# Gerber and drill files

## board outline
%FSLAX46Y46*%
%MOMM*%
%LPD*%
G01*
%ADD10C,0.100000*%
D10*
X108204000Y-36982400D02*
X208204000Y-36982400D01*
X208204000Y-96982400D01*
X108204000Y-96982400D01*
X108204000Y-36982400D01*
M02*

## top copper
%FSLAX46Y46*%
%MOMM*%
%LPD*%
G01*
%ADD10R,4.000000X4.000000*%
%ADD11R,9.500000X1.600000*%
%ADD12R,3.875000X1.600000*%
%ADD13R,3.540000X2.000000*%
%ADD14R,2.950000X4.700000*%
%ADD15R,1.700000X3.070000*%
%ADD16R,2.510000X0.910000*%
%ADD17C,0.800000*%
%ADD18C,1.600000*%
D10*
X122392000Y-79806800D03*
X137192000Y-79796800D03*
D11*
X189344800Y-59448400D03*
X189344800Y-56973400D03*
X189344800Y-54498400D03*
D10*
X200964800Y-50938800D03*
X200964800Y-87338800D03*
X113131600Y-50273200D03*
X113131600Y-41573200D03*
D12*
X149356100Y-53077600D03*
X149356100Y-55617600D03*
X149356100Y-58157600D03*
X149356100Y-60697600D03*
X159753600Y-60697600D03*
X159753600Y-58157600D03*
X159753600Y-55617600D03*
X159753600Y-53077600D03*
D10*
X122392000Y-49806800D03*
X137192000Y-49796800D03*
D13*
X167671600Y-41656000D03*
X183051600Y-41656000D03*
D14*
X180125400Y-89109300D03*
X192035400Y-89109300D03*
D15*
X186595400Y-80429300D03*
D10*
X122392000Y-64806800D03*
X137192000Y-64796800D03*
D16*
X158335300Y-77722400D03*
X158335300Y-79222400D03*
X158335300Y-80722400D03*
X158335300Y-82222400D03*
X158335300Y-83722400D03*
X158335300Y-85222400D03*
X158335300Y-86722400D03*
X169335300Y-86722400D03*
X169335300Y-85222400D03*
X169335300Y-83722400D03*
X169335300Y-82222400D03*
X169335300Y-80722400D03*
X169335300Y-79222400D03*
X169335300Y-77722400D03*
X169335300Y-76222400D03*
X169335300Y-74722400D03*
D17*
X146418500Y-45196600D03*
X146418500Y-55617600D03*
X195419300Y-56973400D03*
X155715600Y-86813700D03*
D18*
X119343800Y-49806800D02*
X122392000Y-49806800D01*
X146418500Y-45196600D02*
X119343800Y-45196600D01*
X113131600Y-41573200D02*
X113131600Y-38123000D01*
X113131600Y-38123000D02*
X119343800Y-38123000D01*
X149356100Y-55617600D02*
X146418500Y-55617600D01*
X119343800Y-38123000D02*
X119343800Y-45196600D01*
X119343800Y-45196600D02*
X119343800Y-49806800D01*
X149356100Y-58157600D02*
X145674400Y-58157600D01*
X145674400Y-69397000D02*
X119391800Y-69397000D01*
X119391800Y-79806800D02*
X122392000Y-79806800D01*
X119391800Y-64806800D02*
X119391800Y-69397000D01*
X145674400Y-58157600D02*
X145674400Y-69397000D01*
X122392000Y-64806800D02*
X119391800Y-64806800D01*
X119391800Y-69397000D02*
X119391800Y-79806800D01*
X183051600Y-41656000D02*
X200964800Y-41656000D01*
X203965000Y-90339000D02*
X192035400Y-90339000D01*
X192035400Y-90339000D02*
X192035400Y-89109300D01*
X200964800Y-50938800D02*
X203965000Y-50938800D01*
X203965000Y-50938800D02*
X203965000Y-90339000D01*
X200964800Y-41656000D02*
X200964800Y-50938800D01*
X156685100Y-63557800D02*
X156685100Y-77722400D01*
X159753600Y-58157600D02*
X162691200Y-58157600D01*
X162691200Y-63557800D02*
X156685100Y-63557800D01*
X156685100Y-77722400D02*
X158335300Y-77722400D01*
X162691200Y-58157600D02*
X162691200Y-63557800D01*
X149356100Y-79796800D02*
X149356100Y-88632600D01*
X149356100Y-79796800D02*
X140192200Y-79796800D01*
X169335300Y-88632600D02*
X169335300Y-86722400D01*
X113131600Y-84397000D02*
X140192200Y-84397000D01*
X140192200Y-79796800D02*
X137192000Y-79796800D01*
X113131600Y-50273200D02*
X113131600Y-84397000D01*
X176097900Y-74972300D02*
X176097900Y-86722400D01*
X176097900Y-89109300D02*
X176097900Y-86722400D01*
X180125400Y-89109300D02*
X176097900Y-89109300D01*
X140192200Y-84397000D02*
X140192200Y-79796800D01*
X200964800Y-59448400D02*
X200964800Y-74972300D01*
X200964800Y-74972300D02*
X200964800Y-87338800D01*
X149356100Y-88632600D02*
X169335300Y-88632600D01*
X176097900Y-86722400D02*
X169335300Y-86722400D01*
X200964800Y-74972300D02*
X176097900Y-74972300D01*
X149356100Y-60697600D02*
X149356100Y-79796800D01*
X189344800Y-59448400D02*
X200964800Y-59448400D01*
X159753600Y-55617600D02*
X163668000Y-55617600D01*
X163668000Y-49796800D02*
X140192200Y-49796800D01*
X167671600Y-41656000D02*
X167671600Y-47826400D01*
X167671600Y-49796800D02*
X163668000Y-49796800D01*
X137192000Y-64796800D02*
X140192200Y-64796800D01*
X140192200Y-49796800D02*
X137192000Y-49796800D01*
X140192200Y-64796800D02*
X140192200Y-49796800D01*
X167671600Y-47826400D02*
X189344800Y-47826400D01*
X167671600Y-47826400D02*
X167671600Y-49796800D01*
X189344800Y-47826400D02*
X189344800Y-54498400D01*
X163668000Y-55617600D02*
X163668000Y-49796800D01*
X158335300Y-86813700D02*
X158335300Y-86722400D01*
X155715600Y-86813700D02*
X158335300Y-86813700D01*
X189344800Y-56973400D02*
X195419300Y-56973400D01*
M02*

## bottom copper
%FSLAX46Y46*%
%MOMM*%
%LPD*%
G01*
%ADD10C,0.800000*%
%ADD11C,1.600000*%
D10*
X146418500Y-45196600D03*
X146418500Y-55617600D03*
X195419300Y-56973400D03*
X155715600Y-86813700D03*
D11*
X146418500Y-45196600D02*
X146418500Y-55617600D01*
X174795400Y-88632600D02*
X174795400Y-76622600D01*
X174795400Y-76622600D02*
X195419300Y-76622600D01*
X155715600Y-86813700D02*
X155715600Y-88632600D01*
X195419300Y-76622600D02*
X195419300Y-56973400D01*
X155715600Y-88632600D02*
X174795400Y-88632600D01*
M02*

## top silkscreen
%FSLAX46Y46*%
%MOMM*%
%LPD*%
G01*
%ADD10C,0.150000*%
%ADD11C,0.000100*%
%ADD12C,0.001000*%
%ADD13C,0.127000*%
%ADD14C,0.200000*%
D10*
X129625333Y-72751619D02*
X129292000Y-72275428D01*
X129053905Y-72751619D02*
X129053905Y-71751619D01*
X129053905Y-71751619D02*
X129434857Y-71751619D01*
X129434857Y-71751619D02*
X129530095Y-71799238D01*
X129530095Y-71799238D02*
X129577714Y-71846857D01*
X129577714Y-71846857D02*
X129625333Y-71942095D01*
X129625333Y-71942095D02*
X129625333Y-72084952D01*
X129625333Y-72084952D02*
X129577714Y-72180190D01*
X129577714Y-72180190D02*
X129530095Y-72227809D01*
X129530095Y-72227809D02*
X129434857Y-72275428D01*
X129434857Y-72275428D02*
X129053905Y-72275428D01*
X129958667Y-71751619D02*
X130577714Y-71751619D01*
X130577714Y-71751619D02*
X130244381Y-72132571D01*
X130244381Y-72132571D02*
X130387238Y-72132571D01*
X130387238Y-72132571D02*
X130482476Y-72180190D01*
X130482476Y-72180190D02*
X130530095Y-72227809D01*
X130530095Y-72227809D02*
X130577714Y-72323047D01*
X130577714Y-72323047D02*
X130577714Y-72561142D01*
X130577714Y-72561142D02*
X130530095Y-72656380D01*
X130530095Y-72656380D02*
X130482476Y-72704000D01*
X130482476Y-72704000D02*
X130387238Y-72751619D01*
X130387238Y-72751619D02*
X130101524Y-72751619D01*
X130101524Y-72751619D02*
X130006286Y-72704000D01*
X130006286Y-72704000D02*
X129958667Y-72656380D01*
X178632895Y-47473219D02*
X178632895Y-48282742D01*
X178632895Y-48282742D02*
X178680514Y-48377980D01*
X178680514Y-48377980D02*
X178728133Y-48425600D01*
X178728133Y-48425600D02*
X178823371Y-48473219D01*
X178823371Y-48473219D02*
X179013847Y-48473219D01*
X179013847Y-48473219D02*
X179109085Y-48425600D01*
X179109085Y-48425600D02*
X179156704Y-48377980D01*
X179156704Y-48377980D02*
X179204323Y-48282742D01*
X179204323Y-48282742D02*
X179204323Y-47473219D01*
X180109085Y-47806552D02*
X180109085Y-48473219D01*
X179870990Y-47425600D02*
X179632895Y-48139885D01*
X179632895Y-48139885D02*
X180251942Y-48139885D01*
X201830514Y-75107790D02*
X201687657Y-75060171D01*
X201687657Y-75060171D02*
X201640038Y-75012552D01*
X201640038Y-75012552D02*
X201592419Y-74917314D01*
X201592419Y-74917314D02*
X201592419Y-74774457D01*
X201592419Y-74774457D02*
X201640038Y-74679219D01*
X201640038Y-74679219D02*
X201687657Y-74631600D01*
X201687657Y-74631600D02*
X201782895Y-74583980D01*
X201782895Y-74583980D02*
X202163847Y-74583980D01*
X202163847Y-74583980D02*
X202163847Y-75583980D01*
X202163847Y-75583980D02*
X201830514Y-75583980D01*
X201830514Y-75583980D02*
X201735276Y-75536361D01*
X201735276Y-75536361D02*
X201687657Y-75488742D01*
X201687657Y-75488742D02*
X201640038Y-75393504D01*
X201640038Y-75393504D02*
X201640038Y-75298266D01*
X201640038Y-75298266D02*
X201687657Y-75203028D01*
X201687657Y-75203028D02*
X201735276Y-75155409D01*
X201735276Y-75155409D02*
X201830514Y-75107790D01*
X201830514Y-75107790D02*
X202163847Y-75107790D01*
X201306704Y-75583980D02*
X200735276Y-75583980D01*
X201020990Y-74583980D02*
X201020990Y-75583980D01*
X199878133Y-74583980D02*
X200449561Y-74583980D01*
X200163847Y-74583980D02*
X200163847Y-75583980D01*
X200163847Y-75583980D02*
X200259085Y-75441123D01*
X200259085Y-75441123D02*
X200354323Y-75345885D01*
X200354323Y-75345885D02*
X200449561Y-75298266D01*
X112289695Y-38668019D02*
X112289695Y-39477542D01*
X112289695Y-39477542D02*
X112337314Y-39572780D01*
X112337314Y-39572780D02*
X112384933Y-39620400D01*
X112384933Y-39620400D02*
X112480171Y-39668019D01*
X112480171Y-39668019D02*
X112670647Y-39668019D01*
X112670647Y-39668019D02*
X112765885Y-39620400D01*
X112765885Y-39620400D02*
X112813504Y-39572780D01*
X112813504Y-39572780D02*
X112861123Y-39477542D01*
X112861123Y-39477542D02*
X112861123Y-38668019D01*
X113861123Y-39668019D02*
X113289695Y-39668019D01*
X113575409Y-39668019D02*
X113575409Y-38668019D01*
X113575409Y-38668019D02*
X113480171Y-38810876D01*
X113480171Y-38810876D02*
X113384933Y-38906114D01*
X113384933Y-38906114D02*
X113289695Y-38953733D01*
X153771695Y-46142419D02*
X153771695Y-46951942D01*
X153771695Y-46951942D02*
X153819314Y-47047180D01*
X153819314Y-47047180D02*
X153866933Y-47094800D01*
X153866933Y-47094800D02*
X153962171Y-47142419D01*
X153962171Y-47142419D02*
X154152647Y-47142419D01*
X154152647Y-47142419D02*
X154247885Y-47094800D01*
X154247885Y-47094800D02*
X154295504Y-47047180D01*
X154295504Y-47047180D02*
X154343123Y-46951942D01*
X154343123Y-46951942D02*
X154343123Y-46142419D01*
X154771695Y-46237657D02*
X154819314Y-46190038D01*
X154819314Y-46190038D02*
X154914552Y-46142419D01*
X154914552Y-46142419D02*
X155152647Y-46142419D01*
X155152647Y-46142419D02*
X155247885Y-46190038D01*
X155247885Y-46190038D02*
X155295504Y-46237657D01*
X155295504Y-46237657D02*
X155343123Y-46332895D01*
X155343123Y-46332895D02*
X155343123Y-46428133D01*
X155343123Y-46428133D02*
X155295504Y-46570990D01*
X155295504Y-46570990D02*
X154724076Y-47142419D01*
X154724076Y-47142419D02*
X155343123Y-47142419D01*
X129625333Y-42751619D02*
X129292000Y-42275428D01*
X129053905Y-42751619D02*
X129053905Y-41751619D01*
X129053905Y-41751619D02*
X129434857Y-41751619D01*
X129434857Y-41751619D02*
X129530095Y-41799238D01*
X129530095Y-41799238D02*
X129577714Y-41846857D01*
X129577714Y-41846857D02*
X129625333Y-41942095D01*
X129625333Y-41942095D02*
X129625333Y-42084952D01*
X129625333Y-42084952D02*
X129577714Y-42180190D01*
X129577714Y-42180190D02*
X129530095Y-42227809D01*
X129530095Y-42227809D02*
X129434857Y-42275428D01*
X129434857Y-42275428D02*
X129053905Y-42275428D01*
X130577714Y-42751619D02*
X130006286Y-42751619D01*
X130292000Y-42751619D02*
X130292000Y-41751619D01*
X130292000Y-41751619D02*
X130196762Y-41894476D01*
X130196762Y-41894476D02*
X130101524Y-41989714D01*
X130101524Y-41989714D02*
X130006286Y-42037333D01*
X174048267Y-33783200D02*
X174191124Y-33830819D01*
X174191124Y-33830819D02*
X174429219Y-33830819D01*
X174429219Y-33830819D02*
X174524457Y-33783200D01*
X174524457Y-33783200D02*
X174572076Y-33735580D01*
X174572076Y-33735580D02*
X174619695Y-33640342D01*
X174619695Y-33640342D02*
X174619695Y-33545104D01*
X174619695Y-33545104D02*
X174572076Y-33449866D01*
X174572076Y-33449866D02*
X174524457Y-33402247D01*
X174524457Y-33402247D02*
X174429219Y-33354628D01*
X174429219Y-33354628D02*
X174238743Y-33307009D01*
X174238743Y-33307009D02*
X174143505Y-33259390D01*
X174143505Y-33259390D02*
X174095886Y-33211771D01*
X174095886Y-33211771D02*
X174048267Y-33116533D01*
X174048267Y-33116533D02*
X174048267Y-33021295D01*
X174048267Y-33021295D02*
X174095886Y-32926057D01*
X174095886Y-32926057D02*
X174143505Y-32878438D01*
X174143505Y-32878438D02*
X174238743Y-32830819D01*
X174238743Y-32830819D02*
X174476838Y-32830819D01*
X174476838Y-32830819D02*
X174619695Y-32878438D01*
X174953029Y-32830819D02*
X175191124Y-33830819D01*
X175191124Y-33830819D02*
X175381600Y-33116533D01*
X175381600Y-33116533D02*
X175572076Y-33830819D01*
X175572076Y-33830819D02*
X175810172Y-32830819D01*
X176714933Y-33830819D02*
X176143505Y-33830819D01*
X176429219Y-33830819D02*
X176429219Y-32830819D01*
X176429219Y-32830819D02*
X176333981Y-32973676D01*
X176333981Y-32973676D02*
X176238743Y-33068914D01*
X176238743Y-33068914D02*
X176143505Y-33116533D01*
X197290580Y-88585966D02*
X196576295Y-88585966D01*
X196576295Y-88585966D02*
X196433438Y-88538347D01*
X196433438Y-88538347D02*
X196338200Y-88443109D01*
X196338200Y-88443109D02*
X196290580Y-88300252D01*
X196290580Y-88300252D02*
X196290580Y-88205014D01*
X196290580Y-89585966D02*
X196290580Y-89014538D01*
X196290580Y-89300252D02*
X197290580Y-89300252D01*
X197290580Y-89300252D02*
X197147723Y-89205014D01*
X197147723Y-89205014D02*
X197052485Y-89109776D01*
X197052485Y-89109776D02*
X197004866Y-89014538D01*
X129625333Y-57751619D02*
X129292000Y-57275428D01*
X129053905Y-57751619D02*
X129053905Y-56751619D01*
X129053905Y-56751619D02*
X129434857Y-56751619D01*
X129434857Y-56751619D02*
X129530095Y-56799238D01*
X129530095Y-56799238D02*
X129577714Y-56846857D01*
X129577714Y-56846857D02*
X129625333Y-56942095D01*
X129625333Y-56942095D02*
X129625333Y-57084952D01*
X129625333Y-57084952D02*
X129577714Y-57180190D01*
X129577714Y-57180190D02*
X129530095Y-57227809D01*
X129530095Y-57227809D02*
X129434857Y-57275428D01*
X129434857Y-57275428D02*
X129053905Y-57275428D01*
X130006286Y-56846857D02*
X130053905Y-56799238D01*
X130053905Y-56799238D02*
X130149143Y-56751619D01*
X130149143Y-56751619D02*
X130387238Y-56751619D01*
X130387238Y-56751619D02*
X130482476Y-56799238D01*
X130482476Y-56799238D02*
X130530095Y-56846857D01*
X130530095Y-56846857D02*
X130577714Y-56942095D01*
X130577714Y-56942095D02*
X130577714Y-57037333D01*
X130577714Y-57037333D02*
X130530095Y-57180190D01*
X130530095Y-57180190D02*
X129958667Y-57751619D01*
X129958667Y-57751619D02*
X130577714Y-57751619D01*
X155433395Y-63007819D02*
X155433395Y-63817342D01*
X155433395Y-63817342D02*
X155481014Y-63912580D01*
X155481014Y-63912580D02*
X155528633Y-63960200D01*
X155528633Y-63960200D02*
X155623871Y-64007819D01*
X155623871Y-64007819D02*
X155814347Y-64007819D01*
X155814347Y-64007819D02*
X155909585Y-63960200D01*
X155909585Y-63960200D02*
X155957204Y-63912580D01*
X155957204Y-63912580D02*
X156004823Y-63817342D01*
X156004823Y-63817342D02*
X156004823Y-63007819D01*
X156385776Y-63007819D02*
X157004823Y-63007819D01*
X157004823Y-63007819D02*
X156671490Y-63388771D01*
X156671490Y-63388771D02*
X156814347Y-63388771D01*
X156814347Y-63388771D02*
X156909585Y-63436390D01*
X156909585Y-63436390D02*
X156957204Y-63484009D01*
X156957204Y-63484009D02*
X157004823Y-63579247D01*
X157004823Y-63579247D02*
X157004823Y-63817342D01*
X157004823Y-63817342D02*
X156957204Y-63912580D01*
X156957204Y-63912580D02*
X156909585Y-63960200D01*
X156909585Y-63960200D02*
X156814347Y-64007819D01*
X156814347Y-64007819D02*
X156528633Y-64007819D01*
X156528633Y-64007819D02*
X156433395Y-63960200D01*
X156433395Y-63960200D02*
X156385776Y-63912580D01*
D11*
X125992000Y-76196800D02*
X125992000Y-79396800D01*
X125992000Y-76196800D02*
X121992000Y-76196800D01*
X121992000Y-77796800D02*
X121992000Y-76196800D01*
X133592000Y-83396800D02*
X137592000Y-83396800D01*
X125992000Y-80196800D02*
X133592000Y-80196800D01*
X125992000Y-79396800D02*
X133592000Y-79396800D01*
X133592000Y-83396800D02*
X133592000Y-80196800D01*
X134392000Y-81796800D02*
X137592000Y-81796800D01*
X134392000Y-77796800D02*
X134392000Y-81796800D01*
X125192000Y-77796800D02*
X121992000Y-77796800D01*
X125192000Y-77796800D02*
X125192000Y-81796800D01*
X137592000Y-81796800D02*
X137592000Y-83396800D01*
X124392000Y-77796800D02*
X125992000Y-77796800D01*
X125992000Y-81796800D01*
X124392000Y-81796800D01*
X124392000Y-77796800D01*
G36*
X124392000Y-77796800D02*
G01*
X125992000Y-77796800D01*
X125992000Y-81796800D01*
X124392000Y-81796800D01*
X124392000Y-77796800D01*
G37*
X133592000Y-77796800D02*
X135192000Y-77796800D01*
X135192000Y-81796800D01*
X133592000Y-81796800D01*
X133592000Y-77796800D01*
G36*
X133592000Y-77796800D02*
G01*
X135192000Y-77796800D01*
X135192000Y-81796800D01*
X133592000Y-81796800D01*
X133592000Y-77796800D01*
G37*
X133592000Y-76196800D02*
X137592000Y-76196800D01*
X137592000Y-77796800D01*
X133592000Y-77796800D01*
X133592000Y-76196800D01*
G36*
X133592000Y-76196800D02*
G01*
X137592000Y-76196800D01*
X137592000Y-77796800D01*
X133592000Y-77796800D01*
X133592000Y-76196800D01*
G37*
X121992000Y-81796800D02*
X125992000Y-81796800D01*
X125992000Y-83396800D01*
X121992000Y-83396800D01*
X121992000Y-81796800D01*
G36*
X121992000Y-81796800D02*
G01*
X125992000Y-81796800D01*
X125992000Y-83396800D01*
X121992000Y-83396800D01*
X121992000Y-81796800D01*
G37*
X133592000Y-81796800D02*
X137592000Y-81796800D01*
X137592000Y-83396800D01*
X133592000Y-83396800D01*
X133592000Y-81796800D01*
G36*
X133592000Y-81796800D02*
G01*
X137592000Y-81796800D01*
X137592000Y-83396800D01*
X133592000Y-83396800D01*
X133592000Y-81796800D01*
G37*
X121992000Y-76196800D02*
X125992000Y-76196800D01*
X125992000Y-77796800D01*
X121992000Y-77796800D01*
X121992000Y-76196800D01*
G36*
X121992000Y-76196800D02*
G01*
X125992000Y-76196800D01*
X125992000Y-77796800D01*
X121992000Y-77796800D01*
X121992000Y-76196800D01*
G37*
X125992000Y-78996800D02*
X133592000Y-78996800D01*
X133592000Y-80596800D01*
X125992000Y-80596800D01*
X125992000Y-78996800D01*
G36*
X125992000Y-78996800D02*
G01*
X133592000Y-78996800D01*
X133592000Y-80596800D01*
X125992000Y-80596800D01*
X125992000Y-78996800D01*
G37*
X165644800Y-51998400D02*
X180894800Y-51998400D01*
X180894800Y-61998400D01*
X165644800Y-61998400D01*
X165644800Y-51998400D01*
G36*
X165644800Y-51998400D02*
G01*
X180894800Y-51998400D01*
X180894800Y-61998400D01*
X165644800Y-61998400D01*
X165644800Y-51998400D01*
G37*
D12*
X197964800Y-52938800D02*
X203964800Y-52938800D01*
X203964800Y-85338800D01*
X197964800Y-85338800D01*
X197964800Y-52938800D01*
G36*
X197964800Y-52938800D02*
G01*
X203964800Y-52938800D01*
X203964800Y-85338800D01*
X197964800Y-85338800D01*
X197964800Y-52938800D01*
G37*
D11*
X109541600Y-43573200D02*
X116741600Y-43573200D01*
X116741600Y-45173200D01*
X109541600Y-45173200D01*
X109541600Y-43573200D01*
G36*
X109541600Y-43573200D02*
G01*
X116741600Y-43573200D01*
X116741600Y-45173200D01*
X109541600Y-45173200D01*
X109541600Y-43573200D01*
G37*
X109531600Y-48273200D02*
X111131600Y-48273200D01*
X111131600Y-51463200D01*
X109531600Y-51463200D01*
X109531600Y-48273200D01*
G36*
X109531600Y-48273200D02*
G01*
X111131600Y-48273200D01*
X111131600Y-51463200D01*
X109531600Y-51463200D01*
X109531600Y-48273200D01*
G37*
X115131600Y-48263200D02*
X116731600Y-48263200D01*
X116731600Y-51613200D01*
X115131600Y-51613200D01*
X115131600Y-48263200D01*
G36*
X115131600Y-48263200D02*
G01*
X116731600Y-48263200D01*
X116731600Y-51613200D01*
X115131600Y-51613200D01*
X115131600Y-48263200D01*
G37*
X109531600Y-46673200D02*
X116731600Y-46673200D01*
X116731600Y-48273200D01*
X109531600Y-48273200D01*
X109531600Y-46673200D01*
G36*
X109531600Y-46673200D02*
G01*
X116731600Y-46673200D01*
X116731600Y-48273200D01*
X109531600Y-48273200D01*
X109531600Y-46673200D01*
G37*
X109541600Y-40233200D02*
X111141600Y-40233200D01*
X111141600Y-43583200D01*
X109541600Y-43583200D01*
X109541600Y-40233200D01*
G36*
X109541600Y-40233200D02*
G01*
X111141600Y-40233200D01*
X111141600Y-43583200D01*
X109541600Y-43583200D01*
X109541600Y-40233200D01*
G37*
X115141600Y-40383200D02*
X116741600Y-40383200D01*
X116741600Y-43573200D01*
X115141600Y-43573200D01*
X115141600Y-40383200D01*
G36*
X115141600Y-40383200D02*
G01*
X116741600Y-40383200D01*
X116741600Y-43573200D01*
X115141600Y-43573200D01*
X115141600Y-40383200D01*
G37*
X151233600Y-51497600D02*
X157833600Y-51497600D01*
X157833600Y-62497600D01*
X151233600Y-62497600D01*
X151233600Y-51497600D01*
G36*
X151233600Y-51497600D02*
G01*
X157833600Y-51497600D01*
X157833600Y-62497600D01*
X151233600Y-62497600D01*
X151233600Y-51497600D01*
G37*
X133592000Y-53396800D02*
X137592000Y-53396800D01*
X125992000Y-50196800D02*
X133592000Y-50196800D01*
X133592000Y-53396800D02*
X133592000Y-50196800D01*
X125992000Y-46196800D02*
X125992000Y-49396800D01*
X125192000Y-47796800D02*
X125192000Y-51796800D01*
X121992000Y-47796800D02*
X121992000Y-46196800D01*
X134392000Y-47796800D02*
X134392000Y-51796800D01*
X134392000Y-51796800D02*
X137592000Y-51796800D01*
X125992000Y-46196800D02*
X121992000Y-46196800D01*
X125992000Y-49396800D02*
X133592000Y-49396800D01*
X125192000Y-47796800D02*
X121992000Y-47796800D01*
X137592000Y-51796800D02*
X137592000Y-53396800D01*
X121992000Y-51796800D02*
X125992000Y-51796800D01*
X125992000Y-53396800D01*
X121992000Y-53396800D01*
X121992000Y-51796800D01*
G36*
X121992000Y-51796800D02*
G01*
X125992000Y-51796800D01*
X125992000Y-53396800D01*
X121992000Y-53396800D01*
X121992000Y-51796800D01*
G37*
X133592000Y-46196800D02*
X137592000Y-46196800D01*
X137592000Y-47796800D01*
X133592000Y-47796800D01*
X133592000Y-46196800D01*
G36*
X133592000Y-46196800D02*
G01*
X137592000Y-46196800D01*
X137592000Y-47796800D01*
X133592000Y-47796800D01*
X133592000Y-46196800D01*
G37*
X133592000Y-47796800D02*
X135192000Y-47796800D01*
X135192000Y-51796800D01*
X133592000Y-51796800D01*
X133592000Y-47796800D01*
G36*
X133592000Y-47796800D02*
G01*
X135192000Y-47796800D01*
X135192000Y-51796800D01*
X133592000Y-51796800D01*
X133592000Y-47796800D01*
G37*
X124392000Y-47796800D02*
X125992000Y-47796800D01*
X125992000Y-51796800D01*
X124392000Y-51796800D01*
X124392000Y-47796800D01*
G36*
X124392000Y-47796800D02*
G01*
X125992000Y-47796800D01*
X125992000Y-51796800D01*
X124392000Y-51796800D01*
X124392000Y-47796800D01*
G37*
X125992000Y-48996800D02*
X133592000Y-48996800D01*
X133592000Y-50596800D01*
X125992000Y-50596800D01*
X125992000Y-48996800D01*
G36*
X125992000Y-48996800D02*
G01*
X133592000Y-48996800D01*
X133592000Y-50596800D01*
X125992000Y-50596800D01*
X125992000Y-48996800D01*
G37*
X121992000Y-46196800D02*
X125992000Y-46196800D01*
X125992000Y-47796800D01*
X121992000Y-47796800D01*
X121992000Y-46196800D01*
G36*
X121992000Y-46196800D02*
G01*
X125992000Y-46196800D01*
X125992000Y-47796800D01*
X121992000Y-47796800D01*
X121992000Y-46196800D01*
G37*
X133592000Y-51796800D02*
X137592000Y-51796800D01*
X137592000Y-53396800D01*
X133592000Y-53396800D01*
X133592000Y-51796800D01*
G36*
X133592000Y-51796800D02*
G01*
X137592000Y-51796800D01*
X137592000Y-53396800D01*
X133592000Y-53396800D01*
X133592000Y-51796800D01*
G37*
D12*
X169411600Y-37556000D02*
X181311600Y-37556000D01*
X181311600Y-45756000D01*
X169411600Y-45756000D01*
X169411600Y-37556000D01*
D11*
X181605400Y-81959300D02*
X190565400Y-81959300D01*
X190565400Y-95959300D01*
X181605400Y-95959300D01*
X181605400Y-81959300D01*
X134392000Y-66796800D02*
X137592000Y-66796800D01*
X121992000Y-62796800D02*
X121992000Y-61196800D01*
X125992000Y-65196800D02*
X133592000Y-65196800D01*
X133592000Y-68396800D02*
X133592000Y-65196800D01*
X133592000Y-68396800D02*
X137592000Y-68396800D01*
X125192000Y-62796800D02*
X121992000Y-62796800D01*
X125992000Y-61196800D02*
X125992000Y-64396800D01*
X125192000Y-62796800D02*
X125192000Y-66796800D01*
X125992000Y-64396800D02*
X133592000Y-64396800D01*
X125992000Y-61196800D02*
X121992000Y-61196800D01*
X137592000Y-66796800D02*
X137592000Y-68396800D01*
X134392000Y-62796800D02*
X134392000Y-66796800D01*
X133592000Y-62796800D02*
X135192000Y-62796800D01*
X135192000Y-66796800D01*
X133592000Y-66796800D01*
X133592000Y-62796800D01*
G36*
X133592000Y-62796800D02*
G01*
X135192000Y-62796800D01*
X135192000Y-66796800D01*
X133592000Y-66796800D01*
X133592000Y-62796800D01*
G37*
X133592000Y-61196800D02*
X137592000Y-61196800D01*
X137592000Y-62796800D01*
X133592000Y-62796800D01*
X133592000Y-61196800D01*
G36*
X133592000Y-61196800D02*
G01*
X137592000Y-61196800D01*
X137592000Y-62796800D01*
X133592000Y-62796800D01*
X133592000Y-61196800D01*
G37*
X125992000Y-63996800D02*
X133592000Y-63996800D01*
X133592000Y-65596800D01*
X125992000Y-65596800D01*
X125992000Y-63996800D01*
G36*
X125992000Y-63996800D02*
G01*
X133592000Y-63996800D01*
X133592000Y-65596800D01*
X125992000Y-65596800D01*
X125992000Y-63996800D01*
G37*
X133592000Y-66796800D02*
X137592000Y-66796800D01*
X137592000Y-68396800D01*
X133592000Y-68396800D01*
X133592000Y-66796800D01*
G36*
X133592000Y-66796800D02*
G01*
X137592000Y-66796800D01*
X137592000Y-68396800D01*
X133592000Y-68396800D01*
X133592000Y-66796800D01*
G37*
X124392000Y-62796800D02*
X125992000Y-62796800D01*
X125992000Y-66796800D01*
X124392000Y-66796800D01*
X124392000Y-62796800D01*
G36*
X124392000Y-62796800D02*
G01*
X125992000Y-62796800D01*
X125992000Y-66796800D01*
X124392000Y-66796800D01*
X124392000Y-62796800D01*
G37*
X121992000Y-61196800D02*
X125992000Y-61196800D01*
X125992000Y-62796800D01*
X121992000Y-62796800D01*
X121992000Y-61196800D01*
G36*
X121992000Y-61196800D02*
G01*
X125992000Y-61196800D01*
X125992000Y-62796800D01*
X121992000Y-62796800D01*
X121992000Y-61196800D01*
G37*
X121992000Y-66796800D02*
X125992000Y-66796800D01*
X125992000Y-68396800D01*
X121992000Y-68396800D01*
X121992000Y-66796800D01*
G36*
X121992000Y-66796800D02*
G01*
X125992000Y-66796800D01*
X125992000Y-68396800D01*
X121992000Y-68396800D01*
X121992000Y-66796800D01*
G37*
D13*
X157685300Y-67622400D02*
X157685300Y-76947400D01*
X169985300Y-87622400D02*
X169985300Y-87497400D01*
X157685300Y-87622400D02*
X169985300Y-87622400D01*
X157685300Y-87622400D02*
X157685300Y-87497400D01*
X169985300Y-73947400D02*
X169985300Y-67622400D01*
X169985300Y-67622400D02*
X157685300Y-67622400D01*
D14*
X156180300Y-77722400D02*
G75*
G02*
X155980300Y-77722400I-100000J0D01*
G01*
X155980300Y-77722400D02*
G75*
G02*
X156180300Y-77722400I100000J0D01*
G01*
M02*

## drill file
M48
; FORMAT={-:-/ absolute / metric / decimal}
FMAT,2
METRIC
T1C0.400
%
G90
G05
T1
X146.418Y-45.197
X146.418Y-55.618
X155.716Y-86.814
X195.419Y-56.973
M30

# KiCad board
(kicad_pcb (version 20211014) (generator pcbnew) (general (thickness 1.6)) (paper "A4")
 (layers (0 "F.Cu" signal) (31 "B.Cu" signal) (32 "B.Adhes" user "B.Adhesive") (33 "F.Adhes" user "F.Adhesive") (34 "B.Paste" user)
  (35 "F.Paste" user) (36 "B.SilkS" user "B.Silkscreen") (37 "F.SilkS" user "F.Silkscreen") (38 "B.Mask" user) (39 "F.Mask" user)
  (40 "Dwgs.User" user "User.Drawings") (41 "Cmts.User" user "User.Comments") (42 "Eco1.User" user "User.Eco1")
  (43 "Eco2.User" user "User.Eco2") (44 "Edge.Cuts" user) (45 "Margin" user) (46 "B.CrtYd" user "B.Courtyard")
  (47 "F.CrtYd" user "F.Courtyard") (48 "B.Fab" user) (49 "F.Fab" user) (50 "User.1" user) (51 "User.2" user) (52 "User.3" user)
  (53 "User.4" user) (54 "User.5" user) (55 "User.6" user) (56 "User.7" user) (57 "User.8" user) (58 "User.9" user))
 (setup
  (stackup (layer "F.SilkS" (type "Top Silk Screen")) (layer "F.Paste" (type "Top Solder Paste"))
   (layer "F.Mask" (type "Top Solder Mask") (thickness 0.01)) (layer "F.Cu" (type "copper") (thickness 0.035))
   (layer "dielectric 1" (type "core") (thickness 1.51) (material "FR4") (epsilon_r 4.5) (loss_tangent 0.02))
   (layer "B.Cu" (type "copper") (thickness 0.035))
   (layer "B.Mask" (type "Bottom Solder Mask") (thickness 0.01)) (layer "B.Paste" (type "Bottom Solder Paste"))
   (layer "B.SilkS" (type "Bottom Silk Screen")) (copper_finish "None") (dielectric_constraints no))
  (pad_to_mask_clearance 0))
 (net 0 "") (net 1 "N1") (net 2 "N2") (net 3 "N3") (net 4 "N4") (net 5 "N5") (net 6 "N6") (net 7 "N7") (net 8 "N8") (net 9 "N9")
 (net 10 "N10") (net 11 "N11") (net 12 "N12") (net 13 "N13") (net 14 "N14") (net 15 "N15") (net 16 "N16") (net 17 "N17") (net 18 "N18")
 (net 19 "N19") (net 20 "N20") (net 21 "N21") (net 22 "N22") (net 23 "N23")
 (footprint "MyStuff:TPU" (layer "F.Cu") (at 129.792 79.7968)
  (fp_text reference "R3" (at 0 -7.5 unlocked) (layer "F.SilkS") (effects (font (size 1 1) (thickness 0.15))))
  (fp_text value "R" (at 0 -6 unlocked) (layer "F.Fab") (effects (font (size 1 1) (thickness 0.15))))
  (fp_line (start -3.8 -3.6) (end -3.8 -0.4) (layer "F.SilkS") (width 0.0001))
  (fp_line (start -3.8 -3.6) (end -7.8 -3.6) (layer "F.SilkS") (width 0.0001))
  (fp_line (start -7.8 -2) (end -7.8 -3.6) (layer "F.SilkS") (width 0.0001))
  (fp_line (start 3.8 3.6) (end 7.8 3.6) (layer "F.SilkS") (width 0.0001))
  (fp_line (start -3.8 0.4) (end 3.8 0.4) (layer "F.SilkS") (width 0.0001))
  (fp_line (start -3.8 -0.4) (end 3.8 -0.4) (layer "F.SilkS") (width 0.0001))
  (fp_line (start 3.8 3.6) (end 3.8 0.4) (layer "F.SilkS") (width 0.0001))
  (fp_line (start 4.6 2) (end 7.8 2) (layer "F.SilkS") (width 0.0001))
  (fp_line (start 4.6 -2) (end 4.6 2) (layer "F.SilkS") (width 0.0001))
  (fp_line (start -4.6 -2) (end -7.8 -2) (layer "F.SilkS") (width 0.0001))
  (fp_line (start -4.6 -2) (end -4.6 2) (layer "F.SilkS") (width 0.0001))
  (fp_line (start 7.8 2) (end 7.8 3.6) (layer "F.SilkS") (width 0.0001))
  (fp_rect (start -5.4 -2) (end -3.8 2) (layer "F.SilkS") (width 0.0001) (fill solid))
  (fp_rect (start 3.8 -2) (end 5.4 2) (layer "F.SilkS") (width 0.0001) (fill solid))
  (fp_rect (start 3.8 -3.6) (end 7.8 -2) (layer "F.SilkS") (width 0.0001) (fill solid))
  (fp_rect (start -7.8 2) (end -3.8 3.6) (layer "F.SilkS") (width 0.0001) (fill solid))
  (fp_rect (start 3.8 2) (end 7.8 3.6) (layer "F.SilkS") (width 0.0001) (fill solid))
  (fp_rect (start -7.8 -3.6) (end -3.8 -2) (layer "F.SilkS") (width 0.0001) (fill solid))
  (fp_rect (start -3.8 -0.8) (end 3.8 0.8) (layer "F.SilkS") (width 0.0001) (fill solid))
  (pad "1" smd rect (at -7.4 0.01) (size 4 4) (layers "F.Cu" "F.Paste" "F.Mask") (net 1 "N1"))
  (pad "2" smd rect (at 7.4 0) (size 4 4) (layers "F.Cu" "F.Paste" "F.Mask") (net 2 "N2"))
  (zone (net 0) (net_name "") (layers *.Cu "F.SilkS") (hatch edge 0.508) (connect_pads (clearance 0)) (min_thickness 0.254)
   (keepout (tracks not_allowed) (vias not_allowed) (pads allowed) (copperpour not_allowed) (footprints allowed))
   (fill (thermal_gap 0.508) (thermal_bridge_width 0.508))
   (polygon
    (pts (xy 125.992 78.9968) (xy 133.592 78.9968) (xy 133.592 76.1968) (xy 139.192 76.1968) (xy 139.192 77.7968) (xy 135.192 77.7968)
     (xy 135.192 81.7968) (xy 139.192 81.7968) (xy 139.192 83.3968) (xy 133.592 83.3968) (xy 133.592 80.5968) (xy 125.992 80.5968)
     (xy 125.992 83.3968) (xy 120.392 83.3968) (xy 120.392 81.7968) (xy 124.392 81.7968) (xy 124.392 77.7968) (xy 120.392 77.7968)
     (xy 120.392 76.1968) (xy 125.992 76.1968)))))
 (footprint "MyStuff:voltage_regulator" (layer "F.Cu") (at 179.3748 57.0484)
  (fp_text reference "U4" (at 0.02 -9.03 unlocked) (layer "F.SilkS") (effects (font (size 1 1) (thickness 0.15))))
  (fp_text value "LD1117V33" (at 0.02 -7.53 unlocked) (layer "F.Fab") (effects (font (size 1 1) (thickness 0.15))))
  (fp_rect (start -13.73 -5.05) (end 1.52 4.95) (layer "F.SilkS") (width 0.0001) (fill solid))
  (pad "1" smd rect (at 9.97 2.4) (size 9.5 1.6) (layers "F.Cu" "F.Paste" "F.Mask") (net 2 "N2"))
  (pad "2" smd rect (at 9.97 -0.075) (size 9.5 1.6) (layers "F.Cu" "F.Paste" "F.Mask") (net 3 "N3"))
  (pad "3" smd rect (at 9.97 -2.55) (size 9.5 1.6) (layers "F.Cu" "F.Paste" "F.Mask") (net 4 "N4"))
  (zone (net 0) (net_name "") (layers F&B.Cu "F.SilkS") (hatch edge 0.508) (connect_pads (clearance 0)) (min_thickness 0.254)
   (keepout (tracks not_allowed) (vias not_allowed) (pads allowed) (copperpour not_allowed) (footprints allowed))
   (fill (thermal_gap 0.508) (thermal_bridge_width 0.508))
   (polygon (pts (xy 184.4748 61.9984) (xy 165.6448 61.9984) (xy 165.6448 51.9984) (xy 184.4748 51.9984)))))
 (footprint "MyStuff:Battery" (layer "F.Cu") (at 200.9648 69.1388 180)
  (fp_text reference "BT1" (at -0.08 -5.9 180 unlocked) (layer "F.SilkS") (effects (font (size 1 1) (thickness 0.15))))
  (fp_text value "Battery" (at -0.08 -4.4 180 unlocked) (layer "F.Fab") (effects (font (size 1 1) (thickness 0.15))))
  (fp_rect (start -3 -16.2) (end 3 16.2) (layer "F.SilkS") (width 0.001) (fill solid))
  (pad "1" smd rect (at 0 18.2 180) (size 4 4) (layers "F.Cu" "F.Paste" "F.Mask") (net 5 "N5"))
  (pad "2" smd rect (at 0 -18.2 180) (size 4 4) (layers "F.Cu" "F.Paste" "F.Mask") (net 2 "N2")))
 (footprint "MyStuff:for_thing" (layer "F.Cu") (at 113.1316 45.9232)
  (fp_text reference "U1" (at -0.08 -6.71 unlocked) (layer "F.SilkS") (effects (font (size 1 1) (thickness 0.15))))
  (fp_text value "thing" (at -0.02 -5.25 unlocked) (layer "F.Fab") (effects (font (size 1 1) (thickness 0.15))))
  (fp_rect (start 3.61 -0.75) (end -3.59 -2.35) (layer "F.SilkS") (width 0.0001) (fill solid))
  (fp_rect (start -2 2.35) (end -3.6 5.54) (layer "F.SilkS") (width 0.0001) (fill solid))
  (fp_rect (start 3.6 2.34) (end 2 5.69) (layer "F.SilkS") (width 0.0001) (fill solid))
  (fp_rect (start -3.6 0.75) (end 3.6 2.35) (layer "F.SilkS") (width 0.0001) (fill solid))
  (fp_rect (start -3.59 -2.34) (end -1.99 -5.69) (layer "F.SilkS") (width 0.0001) (fill solid))
  (fp_rect (start 2.01 -2.35) (end 3.61 -5.54) (layer "F.SilkS") (width 0.0001) (fill solid))
  (pad "1" smd rect (at 0 4.35) (size 4 4) (layers "F.Cu" "F.Paste" "F.Mask") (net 2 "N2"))
  (pad "2" smd rect (at 0 -4.35 180) (size 4 4) (layers "F.Cu" "F.Paste" "F.Mask") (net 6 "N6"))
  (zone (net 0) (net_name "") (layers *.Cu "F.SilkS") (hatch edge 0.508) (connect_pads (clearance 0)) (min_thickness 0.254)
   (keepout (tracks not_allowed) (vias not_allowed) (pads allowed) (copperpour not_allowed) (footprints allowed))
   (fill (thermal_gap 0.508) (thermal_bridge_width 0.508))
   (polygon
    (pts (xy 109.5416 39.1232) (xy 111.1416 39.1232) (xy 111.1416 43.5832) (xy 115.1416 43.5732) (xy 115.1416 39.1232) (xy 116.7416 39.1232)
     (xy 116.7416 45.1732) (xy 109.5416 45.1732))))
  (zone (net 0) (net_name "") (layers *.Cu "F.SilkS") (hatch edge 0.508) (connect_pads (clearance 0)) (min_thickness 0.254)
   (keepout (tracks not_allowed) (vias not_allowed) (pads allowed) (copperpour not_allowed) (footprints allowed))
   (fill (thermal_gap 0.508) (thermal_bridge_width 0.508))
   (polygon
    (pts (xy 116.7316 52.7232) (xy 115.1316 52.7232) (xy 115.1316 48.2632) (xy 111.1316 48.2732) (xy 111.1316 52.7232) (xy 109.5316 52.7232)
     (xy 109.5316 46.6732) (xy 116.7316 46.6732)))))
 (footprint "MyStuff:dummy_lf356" (layer "F.Cu") (at 154.5336 56.9976)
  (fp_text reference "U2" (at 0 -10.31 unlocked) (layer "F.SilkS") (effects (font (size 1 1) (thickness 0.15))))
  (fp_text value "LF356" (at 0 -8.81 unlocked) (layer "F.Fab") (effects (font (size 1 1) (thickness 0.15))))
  (fp_rect (start -3.3 -5.5) (end 3.3 5.5) (layer "F.SilkS") (width 0.0001) (fill solid))
  (pad "1" smd rect (at -5.1775 -3.92) (size 3.875 1.6) (layers "F.Cu" "F.Paste" "F.Mask") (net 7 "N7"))
  (pad "2" smd rect (at -5.1775 -1.38) (size 3.875 1.6) (layers "F.Cu" "F.Paste" "F.Mask") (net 6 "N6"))
  (pad "3" smd rect (at -5.1775 1.16) (size 3.875 1.6) (layers "F.Cu" "F.Paste" "F.Mask") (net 1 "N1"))
  (pad "4" smd rect (at -5.1775 3.7) (size 3.875 1.6) (layers "F.Cu" "F.Paste" "F.Mask") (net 2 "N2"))
  (pad "5" smd rect (at 5.22 3.7) (size 3.875 1.6) (layers "F.Cu" "F.Paste" "F.Mask") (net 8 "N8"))
  (pad "6" smd rect (at 5.22 1.16) (size 3.875 1.6) (layers "F.Cu" "F.Paste" "F.Mask") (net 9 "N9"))
  (pad "7" smd rect (at 5.22 -1.38) (size 3.875 1.6) (layers "F.Cu" "F.Paste" "F.Mask") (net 4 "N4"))
  (pad "8" smd rect (at 5.22 -3.92) (size 3.875 1.6) (layers "F.Cu" "F.Paste" "F.Mask") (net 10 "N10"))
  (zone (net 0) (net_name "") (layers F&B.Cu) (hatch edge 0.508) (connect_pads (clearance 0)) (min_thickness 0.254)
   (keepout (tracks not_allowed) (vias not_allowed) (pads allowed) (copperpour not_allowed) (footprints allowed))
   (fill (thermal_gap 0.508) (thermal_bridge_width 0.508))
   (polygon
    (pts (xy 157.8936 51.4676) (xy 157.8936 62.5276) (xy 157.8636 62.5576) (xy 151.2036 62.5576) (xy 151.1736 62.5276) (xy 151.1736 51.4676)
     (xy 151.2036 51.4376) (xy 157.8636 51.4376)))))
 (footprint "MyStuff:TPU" (layer "F.Cu") (at 129.792 49.7968)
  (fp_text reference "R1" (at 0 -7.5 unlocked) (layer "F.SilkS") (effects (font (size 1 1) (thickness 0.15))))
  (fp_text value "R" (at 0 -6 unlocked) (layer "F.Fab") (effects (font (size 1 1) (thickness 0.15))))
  (fp_line (start 3.8 3.6) (end 7.8 3.6) (layer "F.SilkS") (width 0.0001))
  (fp_line (start -3.8 0.4) (end 3.8 0.4) (layer "F.SilkS") (width 0.0001))
  (fp_line (start 3.8 3.6) (end 3.8 0.4) (layer "F.SilkS") (width 0.0001))
  (fp_line (start -3.8 -3.6) (end -3.8 -0.4) (layer "F.SilkS") (width 0.0001))
  (fp_line (start -4.6 -2) (end -4.6 2) (layer "F.SilkS") (width 0.0001))
  (fp_line (start -7.8 -2) (end -7.8 -3.6) (layer "F.SilkS") (width 0.0001))
  (fp_line (start 4.6 -2) (end 4.6 2) (layer "F.SilkS") (width 0.0001))
  (fp_line (start 4.6 2) (end 7.8 2) (layer "F.SilkS") (width 0.0001))
  (fp_line (start -3.8 -3.6) (end -7.8 -3.6) (layer "F.SilkS") (width 0.0001))
  (fp_line (start -3.8 -0.4) (end 3.8 -0.4) (layer "F.SilkS") (width 0.0001))
  (fp_line (start -4.6 -2) (end -7.8 -2) (layer "F.SilkS") (width 0.0001))
  (fp_line (start 7.8 2) (end 7.8 3.6) (layer "F.SilkS") (width 0.0001))
  (fp_rect (start -7.8 2) (end -3.8 3.6) (layer "F.SilkS") (width 0.0001) (fill solid))
  (fp_rect (start 3.8 -3.6) (end 7.8 -2) (layer "F.SilkS") (width 0.0001) (fill solid))
  (fp_rect (start 3.8 -2) (end 5.4 2) (layer "F.SilkS") (width 0.0001) (fill solid))
  (fp_rect (start -5.4 -2) (end -3.8 2) (layer "F.SilkS") (width 0.0001) (fill solid))
  (fp_rect (start -3.8 -0.8) (end 3.8 0.8) (layer "F.SilkS") (width 0.0001) (fill solid))
  (fp_rect (start -7.8 -3.6) (end -3.8 -2) (layer "F.SilkS") (width 0.0001) (fill solid))
  (fp_rect (start 3.8 2) (end 7.8 3.6) (layer "F.SilkS") (width 0.0001) (fill solid))
  (pad "1" smd rect (at -7.4 0.01) (size 4 4) (layers "F.Cu" "F.Paste" "F.Mask") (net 6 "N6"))
  (pad "2" smd rect (at 7.4 0) (size 4 4) (layers "F.Cu" "F.Paste" "F.Mask") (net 4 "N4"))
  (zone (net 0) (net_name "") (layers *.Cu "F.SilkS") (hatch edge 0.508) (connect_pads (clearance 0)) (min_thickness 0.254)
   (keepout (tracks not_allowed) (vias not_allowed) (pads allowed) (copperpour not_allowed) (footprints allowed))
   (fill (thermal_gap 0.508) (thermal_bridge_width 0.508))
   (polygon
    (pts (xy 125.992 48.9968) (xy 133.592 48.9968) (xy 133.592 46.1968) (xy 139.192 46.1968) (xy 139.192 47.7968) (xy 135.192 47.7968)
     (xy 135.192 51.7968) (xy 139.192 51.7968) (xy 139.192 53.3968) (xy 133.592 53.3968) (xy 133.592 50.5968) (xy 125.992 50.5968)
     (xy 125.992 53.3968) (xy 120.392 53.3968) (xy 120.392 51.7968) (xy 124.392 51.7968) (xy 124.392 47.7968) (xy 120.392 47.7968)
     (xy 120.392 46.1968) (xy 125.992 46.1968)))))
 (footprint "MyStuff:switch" (layer "F.Cu") (at 175.3616 41.656)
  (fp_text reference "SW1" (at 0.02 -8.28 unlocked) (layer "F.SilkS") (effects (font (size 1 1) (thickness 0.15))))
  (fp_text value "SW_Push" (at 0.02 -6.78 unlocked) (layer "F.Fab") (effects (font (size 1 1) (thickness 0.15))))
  (fp_rect (start -5.95 4.1) (end 5.95 -4.1) (layer "F.SilkS") (width 0.001) (fill none))
  (pad "1" smd rect (at -7.69 0) (size 3.54 2) (layers "F.Cu" "F.Paste" "F.Mask") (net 4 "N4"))
  (pad "2" smd rect (at 7.69 0) (size 3.54 2) (layers "F.Cu" "F.Paste" "F.Mask") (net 5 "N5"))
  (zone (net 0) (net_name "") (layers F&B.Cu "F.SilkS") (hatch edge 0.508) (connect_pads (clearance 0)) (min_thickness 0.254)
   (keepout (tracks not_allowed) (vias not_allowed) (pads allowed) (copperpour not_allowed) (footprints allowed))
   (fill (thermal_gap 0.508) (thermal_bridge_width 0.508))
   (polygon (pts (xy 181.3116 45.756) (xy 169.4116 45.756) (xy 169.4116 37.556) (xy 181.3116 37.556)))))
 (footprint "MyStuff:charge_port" (layer "F.Cu") (at 186.0854 88.9593 -90)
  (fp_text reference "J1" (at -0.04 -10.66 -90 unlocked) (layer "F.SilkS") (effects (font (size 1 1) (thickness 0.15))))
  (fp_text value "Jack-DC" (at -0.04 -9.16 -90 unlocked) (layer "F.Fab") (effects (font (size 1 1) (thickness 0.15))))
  (fp_rect (start -7 -4.48) (end 7 4.48) (layer "F.SilkS") (width 0.0001) (fill none))
  (pad "1" smd rect (at 0.15 5.96 90) (size 4.7 2.95) (layers "F.Cu" "F.Paste" "F.Mask") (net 2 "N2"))
  (pad "2" smd rect (at 0.15 -5.95 90) (size 4.7 2.95) (layers "F.Cu" "F.Paste" "F.Mask") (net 5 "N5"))
  (pad "3" smd rect (at -8.53 -0.51 90) (size 3.07 1.7) (layers "F.Cu" "F.Paste" "F.Mask")))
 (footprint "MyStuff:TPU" (layer "F.Cu") (at 129.792 64.7968)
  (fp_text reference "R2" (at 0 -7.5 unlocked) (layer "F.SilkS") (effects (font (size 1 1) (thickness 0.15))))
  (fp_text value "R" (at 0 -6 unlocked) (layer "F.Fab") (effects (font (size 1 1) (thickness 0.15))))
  (fp_line (start 4.6 2) (end 7.8 2) (layer "F.SilkS") (width 0.0001))
  (fp_line (start -7.8 -2) (end -7.8 -3.6) (layer "F.SilkS") (width 0.0001))
  (fp_line (start -3.8 0.4) (end 3.8 0.4) (layer "F.SilkS") (width 0.0001))
  (fp_line (start 3.8 3.6) (end 3.8 0.4) (layer "F.SilkS") (width 0.0001))
  (fp_line (start 3.8 3.6) (end 7.8 3.6) (layer "F.SilkS") (width 0.0001))
  (fp_line (start -4.6 -2) (end -7.8 -2) (layer "F.SilkS") (width 0.0001))
  (fp_line (start -3.8 -3.6) (end -3.8 -0.4) (layer "F.SilkS") (width 0.0001))
  (fp_line (start -4.6 -2) (end -4.6 2) (layer "F.SilkS") (width 0.0001))
  (fp_line (start -3.8 -0.4) (end 3.8 -0.4) (layer "F.SilkS") (width 0.0001))
  (fp_line (start -3.8 -3.6) (end -7.8 -3.6) (layer "F.SilkS") (width 0.0001))
  (fp_line (start 7.8 2) (end 7.8 3.6) (layer "F.SilkS") (width 0.0001))
  (fp_line (start 4.6 -2) (end 4.6 2) (layer "F.SilkS") (width 0.0001))
  (fp_rect (start 3.8 -2) (end 5.4 2) (layer "F.SilkS") (width 0.0001) (fill solid))
  (fp_rect (start 3.8 -3.6) (end 7.8 -2) (layer "F.SilkS") (width 0.0001) (fill solid))
  (fp_rect (start -3.8 -0.8) (end 3.8 0.8) (layer "F.SilkS") (width 0.0001) (fill solid))
  (fp_rect (start 3.8 2) (end 7.8 3.6) (layer "F.SilkS") (width 0.0001) (fill solid))
  (fp_rect (start -5.4 -2) (end -3.8 2) (layer "F.SilkS") (width 0.0001) (fill solid))
  (fp_rect (start -7.8 -3.6) (end -3.8 -2) (layer "F.SilkS") (width 0.0001) (fill solid))
  (fp_rect (start -7.8 2) (end -3.8 3.6) (layer "F.SilkS") (width 0.0001) (fill solid))
  (pad "1" smd rect (at -7.4 0.01) (size 4 4) (layers "F.Cu" "F.Paste" "F.Mask") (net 1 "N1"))
  (pad "2" smd rect (at 7.4 0) (size 4 4) (layers "F.Cu" "F.Paste" "F.Mask") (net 4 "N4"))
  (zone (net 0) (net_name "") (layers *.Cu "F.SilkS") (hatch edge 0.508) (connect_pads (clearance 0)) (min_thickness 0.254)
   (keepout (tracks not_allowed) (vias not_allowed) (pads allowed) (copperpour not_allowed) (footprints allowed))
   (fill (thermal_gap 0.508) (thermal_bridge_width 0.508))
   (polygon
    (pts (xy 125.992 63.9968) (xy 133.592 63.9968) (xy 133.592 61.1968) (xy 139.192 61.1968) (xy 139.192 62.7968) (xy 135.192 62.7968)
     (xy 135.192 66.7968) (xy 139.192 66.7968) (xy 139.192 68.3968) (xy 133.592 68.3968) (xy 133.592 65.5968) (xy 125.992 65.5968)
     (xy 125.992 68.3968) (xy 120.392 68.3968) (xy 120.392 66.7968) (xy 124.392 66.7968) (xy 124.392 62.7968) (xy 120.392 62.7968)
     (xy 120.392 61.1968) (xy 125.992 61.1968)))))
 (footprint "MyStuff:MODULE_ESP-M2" (layer "F.Cu") (at 163.8353 77.6224)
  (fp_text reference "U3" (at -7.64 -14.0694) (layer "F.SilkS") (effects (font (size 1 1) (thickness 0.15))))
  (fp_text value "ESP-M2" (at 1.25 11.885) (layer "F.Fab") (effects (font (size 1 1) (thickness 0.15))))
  (fp_line (start -6.15 -10) (end -6.15 -0.675) (layer "F.SilkS") (width 0.127))
  (fp_line (start 6.15 10) (end 6.15 9.875) (layer "F.SilkS") (width 0.127))
  (fp_line (start -6.15 10) (end 6.15 10) (layer "F.SilkS") (width 0.127))
  (fp_line (start -6.15 10) (end -6.15 9.875) (layer "F.SilkS") (width 0.127))
  (fp_line (start 6.15 -3.675) (end 6.15 -10) (layer "F.SilkS") (width 0.127))
  (fp_line (start 6.15 -10) (end -6.15 -10) (layer "F.SilkS") (width 0.127))
  (fp_circle (center -7.755 0.1) (end -7.655 0.1) (layer "F.SilkS") (width 0.2) (fill none))
  (pad "1" smd rect (at -5.5 0.1) (size 2.51 0.91) (layers "F.Cu" "F.Paste" "F.Mask") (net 9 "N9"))
  (pad "2" smd rect (at -5.5 1.6) (size 2.51 0.91) (layers "F.Cu" "F.Paste" "F.Mask") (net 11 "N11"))
  (pad "3" smd rect (at -5.5 3.1) (size 2.51 0.91) (layers "F.Cu" "F.Paste" "F.Mask") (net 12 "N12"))
  (pad "4" smd rect (at -5.5 4.6) (size 2.51 0.91) (layers "F.Cu" "F.Paste" "F.Mask") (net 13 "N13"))
  (pad "5" smd rect (at -5.5 6.1) (size 2.51 0.91) (layers "F.Cu" "F.Paste" "F.Mask") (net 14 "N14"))
  (pad "6" smd rect (at -5.5 7.6) (size 2.51 0.91) (layers "F.Cu" "F.Paste" "F.Mask") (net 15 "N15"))
  (pad "7" smd rect (at -5.5 9.1) (size 2.51 0.91) (layers "F.Cu" "F.Paste" "F.Mask") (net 3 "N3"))
  (pad "8" smd rect (at 5.5 9.1) (size 2.51 0.91) (layers "F.Cu" "F.Paste" "F.Mask") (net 2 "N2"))
  (pad "9" smd rect (at 5.5 7.6) (size 2.51 0.91) (layers "F.Cu" "F.Paste" "F.Mask") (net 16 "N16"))
  (pad "10" smd rect (at 5.5 6.1) (size 2.51 0.91) (layers "F.Cu" "F.Paste" "F.Mask") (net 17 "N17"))
  (pad "11" smd rect (at 5.5 4.6) (size 2.51 0.91) (layers "F.Cu" "F.Paste" "F.Mask") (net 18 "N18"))
  (pad "12" smd rect (at 5.5 3.1) (size 2.51 0.91) (layers "F.Cu" "F.Paste" "F.Mask") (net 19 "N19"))
  (pad "13" smd rect (at 5.5 1.6) (size 2.51 0.91) (layers "F.Cu" "F.Paste" "F.Mask") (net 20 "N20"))
  (pad "14" smd rect (at 5.5 0.1) (size 2.51 0.91) (layers "F.Cu" "F.Paste" "F.Mask") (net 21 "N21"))
  (pad "15" smd rect (at 5.5 -1.4) (size 2.51 0.91) (layers "F.Cu" "F.Paste" "F.Mask") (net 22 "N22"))
  (pad "16" smd rect (at 5.5 -2.9) (size 2.51 0.91) (layers "F.Cu" "F.Paste" "F.Mask") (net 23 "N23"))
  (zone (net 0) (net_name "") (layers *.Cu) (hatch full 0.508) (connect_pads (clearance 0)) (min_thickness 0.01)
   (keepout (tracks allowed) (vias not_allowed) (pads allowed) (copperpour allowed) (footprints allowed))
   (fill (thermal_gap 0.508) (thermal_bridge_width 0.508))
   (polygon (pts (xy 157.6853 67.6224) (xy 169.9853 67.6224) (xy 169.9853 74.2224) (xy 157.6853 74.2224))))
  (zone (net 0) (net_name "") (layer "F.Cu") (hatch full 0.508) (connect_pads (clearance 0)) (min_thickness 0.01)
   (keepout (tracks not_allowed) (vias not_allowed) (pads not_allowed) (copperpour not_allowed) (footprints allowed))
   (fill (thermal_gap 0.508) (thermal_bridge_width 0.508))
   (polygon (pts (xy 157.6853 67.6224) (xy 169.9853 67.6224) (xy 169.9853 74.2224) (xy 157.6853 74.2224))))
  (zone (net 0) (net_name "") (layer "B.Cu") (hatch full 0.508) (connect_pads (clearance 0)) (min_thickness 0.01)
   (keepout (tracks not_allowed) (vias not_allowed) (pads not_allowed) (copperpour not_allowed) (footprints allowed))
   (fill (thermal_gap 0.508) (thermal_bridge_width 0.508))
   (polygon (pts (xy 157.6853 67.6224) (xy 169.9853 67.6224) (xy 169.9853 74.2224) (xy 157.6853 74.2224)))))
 (gr_rect (start 108.204 36.9824) (end 208.204 96.9824) (layer "Edge.Cuts") (width 0.1) (fill none))
 (segment (start 119.3438 49.8068) (end 122.392 49.8068) (width 1.6) (layer "F.Cu") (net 6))
 (segment (start 146.4185 45.1966) (end 119.3438 45.1966) (width 1.6) (layer "F.Cu") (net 6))
 (segment (start 113.1316 41.5732) (end 113.1316 38.123) (width 1.6) (layer "F.Cu") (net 6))
 (segment (start 113.1316 38.123) (end 119.3438 38.123) (width 1.6) (layer "F.Cu") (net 6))
 (segment (start 149.3561 55.6176) (end 146.4185 55.6176) (width 1.6) (layer "F.Cu") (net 6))
 (segment (start 119.3438 38.123) (end 119.3438 45.1966) (width 1.6) (layer "F.Cu") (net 6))
 (segment (start 119.3438 45.1966) (end 119.3438 49.8068) (width 1.6) (layer "F.Cu") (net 6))
 (via (at 146.4185 45.1966) (size 0.8) (drill 0.4) (layers "F.Cu" "B.Cu") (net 6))
 (via (at 146.4185 55.6176) (size 0.8) (drill 0.4) (layers "F.Cu" "B.Cu") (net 6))
 (segment (start 146.4185 45.1966) (end 146.4185 55.6176) (width 1.6) (layer "B.Cu") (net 6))
 (segment (start 149.3561 58.1576) (end 145.6744 58.1576) (width 1.6) (layer "F.Cu") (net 1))
 (segment (start 145.6744 69.397) (end 119.3918 69.397) (width 1.6) (layer "F.Cu") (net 1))
 (segment (start 119.3918 79.8068) (end 122.392 79.8068) (width 1.6) (layer "F.Cu") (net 1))
 (segment (start 119.3918 64.8068) (end 119.3918 69.397) (width 1.6) (layer "F.Cu") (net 1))
 (segment (start 145.6744 58.1576) (end 145.6744 69.397) (width 1.6) (layer "F.Cu") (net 1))
 (segment (start 122.392 64.8068) (end 119.3918 64.8068) (width 1.6) (layer "F.Cu") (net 1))
 (segment (start 119.3918 69.397) (end 119.3918 79.8068) (width 1.6) (layer "F.Cu") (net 1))
 (segment (start 183.0516 41.656) (end 200.9648 41.656) (width 1.6) (layer "F.Cu") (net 5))
 (segment (start 203.965 90.339) (end 192.0354 90.339) (width 1.6) (layer "F.Cu") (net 5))
 (segment (start 192.0354 90.339) (end 192.0354 89.1093) (width 1.6) (layer "F.Cu") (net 5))
 (segment (start 200.9648 50.9388) (end 203.965 50.9388) (width 1.6) (layer "F.Cu") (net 5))
 (segment (start 203.965 50.9388) (end 203.965 90.339) (width 1.6) (layer "F.Cu") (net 5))
 (segment (start 200.9648 41.656) (end 200.9648 50.9388) (width 1.6) (layer "F.Cu") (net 5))
 (segment (start 156.6851 63.5578) (end 156.6851 77.7224) (width 1.6) (layer "F.Cu") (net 9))
 (segment (start 159.7536 58.1576) (end 162.6912 58.1576) (width 1.6) (layer "F.Cu") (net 9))
 (segment (start 162.6912 63.5578) (end 156.6851 63.5578) (width 1.6) (layer "F.Cu") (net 9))
 (segment (start 156.6851 77.7224) (end 158.3353 77.7224) (width 1.6) (layer "F.Cu") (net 9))
 (segment (start 162.6912 58.1576) (end 162.6912 63.5578) (width 1.6) (layer "F.Cu") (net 9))
 (segment (start 149.3561 79.7968) (end 149.3561 88.6326) (width 1.6) (layer "F.Cu") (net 2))
 (segment (start 149.3561 79.7968) (end 140.1922 79.7968) (width 1.6) (layer "F.Cu") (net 2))
 (segment (start 169.3353 88.6326) (end 169.3353 86.7224) (width 1.6) (layer "F.Cu") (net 2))
 (segment (start 113.1316 84.397) (end 140.1922 84.397) (width 1.6) (layer "F.Cu") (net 2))
 (segment (start 140.1922 79.7968) (end 137.192 79.7968) (width 1.6) (layer "F.Cu") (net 2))
 (segment (start 113.1316 50.2732) (end 113.1316 84.397) (width 1.6) (layer "F.Cu") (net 2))
 (segment (start 176.0979 74.9723) (end 176.0979 86.7224) (width 1.6) (layer "F.Cu") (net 2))
 (segment (start 176.0979 89.1093) (end 176.0979 86.7224) (width 1.6) (layer "F.Cu") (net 2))
 (segment (start 180.1254 89.1093) (end 176.0979 89.1093) (width 1.6) (layer "F.Cu") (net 2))
 (segment (start 140.1922 84.397) (end 140.1922 79.7968) (width 1.6) (layer "F.Cu") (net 2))
 (segment (start 200.9648 59.4484) (end 200.9648 74.9723) (width 1.6) (layer "F.Cu") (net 2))
 (segment (start 200.9648 74.9723) (end 200.9648 87.3388) (width 1.6) (layer "F.Cu") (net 2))
 (segment (start 149.3561 88.6326) (end 169.3353 88.6326) (width 1.6) (layer "F.Cu") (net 2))
 (segment (start 176.0979 86.7224) (end 169.3353 86.7224) (width 1.6) (layer "F.Cu") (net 2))
 (segment (start 200.9648 74.9723) (end 176.0979 74.9723) (width 1.6) (layer "F.Cu") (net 2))
 (segment (start 149.3561 60.6976) (end 149.3561 79.7968) (width 1.6) (layer "F.Cu") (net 2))
 (segment (start 189.3448 59.4484) (end 200.9648 59.4484) (width 1.6) (layer "F.Cu") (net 2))
 (segment (start 159.7536 55.6176) (end 163.668 55.6176) (width 1.6) (layer "F.Cu") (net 4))
 (segment (start 163.668 49.7968) (end 140.1922 49.7968) (width 1.6) (layer "F.Cu") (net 4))
 (segment (start 167.6716 41.656) (end 167.6716 47.8264) (width 1.6) (layer "F.Cu") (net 4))
 (segment (start 167.6716 49.7968) (end 163.668 49.7968) (width 1.6) (layer "F.Cu") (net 4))
 (segment (start 137.192 64.7968) (end 140.1922 64.7968) (width 1.6) (layer "F.Cu") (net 4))
 (segment (start 140.1922 49.7968) (end 137.192 49.7968) (width 1.6) (layer "F.Cu") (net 4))
 (segment (start 140.1922 64.7968) (end 140.1922 49.7968) (width 1.6) (layer "F.Cu") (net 4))
 (segment (start 167.6716 47.8264) (end 189.3448 47.8264) (width 1.6) (layer "F.Cu") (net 4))
 (segment (start 167.6716 47.8264) (end 167.6716 49.7968) (width 1.6) (layer "F.Cu") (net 4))
 (segment (start 189.3448 47.8264) (end 189.3448 54.4984) (width 1.6) (layer "F.Cu") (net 4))
 (segment (start 163.668 55.6176) (end 163.668 49.7968) (width 1.6) (layer "F.Cu") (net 4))
 (segment (start 158.3353 86.8137) (end 158.3353 86.7224) (width 1.6) (layer "F.Cu") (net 3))
 (segment (start 155.7156 86.8137) (end 158.3353 86.8137) (width 1.6) (layer "F.Cu") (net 3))
 (segment (start 189.3448 56.9734) (end 195.4193 56.9734) (width 1.6) (layer "F.Cu") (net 3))
 (via (at 195.4193 56.9734) (size 0.8) (drill 0.4) (layers "F.Cu" "B.Cu") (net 3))
 (via (at 155.7156 86.8137) (size 0.8) (drill 0.4) (layers "F.Cu" "B.Cu") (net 3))
 (segment (start 174.7954 88.6326) (end 174.7954 76.6226) (width 1.6) (layer "B.Cu") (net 3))
 (segment (start 174.7954 76.6226) (end 195.4193 76.6226) (width 1.6) (layer "B.Cu") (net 3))
 (segment (start 155.7156 86.8137) (end 155.7156 88.6326) (width 1.6) (layer "B.Cu") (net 3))
 (segment (start 195.4193 76.6226) (end 195.4193 56.9734) (width 1.6) (layer "B.Cu") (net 3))
 (segment (start 155.7156 88.6326) (end 174.7954 88.6326) (width 1.6) (layer "B.Cu") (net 3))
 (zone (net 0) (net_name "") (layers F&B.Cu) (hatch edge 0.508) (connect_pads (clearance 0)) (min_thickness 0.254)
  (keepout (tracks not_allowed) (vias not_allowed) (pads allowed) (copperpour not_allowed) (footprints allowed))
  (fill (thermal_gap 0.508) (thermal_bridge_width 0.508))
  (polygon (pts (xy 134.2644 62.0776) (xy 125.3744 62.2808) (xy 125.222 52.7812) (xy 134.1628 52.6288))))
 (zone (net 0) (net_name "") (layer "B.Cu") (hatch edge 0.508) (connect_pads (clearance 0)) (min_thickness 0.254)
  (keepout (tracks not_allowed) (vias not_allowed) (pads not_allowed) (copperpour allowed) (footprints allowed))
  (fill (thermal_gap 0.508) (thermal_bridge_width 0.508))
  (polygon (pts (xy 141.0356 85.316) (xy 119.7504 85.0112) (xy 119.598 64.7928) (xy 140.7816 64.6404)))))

